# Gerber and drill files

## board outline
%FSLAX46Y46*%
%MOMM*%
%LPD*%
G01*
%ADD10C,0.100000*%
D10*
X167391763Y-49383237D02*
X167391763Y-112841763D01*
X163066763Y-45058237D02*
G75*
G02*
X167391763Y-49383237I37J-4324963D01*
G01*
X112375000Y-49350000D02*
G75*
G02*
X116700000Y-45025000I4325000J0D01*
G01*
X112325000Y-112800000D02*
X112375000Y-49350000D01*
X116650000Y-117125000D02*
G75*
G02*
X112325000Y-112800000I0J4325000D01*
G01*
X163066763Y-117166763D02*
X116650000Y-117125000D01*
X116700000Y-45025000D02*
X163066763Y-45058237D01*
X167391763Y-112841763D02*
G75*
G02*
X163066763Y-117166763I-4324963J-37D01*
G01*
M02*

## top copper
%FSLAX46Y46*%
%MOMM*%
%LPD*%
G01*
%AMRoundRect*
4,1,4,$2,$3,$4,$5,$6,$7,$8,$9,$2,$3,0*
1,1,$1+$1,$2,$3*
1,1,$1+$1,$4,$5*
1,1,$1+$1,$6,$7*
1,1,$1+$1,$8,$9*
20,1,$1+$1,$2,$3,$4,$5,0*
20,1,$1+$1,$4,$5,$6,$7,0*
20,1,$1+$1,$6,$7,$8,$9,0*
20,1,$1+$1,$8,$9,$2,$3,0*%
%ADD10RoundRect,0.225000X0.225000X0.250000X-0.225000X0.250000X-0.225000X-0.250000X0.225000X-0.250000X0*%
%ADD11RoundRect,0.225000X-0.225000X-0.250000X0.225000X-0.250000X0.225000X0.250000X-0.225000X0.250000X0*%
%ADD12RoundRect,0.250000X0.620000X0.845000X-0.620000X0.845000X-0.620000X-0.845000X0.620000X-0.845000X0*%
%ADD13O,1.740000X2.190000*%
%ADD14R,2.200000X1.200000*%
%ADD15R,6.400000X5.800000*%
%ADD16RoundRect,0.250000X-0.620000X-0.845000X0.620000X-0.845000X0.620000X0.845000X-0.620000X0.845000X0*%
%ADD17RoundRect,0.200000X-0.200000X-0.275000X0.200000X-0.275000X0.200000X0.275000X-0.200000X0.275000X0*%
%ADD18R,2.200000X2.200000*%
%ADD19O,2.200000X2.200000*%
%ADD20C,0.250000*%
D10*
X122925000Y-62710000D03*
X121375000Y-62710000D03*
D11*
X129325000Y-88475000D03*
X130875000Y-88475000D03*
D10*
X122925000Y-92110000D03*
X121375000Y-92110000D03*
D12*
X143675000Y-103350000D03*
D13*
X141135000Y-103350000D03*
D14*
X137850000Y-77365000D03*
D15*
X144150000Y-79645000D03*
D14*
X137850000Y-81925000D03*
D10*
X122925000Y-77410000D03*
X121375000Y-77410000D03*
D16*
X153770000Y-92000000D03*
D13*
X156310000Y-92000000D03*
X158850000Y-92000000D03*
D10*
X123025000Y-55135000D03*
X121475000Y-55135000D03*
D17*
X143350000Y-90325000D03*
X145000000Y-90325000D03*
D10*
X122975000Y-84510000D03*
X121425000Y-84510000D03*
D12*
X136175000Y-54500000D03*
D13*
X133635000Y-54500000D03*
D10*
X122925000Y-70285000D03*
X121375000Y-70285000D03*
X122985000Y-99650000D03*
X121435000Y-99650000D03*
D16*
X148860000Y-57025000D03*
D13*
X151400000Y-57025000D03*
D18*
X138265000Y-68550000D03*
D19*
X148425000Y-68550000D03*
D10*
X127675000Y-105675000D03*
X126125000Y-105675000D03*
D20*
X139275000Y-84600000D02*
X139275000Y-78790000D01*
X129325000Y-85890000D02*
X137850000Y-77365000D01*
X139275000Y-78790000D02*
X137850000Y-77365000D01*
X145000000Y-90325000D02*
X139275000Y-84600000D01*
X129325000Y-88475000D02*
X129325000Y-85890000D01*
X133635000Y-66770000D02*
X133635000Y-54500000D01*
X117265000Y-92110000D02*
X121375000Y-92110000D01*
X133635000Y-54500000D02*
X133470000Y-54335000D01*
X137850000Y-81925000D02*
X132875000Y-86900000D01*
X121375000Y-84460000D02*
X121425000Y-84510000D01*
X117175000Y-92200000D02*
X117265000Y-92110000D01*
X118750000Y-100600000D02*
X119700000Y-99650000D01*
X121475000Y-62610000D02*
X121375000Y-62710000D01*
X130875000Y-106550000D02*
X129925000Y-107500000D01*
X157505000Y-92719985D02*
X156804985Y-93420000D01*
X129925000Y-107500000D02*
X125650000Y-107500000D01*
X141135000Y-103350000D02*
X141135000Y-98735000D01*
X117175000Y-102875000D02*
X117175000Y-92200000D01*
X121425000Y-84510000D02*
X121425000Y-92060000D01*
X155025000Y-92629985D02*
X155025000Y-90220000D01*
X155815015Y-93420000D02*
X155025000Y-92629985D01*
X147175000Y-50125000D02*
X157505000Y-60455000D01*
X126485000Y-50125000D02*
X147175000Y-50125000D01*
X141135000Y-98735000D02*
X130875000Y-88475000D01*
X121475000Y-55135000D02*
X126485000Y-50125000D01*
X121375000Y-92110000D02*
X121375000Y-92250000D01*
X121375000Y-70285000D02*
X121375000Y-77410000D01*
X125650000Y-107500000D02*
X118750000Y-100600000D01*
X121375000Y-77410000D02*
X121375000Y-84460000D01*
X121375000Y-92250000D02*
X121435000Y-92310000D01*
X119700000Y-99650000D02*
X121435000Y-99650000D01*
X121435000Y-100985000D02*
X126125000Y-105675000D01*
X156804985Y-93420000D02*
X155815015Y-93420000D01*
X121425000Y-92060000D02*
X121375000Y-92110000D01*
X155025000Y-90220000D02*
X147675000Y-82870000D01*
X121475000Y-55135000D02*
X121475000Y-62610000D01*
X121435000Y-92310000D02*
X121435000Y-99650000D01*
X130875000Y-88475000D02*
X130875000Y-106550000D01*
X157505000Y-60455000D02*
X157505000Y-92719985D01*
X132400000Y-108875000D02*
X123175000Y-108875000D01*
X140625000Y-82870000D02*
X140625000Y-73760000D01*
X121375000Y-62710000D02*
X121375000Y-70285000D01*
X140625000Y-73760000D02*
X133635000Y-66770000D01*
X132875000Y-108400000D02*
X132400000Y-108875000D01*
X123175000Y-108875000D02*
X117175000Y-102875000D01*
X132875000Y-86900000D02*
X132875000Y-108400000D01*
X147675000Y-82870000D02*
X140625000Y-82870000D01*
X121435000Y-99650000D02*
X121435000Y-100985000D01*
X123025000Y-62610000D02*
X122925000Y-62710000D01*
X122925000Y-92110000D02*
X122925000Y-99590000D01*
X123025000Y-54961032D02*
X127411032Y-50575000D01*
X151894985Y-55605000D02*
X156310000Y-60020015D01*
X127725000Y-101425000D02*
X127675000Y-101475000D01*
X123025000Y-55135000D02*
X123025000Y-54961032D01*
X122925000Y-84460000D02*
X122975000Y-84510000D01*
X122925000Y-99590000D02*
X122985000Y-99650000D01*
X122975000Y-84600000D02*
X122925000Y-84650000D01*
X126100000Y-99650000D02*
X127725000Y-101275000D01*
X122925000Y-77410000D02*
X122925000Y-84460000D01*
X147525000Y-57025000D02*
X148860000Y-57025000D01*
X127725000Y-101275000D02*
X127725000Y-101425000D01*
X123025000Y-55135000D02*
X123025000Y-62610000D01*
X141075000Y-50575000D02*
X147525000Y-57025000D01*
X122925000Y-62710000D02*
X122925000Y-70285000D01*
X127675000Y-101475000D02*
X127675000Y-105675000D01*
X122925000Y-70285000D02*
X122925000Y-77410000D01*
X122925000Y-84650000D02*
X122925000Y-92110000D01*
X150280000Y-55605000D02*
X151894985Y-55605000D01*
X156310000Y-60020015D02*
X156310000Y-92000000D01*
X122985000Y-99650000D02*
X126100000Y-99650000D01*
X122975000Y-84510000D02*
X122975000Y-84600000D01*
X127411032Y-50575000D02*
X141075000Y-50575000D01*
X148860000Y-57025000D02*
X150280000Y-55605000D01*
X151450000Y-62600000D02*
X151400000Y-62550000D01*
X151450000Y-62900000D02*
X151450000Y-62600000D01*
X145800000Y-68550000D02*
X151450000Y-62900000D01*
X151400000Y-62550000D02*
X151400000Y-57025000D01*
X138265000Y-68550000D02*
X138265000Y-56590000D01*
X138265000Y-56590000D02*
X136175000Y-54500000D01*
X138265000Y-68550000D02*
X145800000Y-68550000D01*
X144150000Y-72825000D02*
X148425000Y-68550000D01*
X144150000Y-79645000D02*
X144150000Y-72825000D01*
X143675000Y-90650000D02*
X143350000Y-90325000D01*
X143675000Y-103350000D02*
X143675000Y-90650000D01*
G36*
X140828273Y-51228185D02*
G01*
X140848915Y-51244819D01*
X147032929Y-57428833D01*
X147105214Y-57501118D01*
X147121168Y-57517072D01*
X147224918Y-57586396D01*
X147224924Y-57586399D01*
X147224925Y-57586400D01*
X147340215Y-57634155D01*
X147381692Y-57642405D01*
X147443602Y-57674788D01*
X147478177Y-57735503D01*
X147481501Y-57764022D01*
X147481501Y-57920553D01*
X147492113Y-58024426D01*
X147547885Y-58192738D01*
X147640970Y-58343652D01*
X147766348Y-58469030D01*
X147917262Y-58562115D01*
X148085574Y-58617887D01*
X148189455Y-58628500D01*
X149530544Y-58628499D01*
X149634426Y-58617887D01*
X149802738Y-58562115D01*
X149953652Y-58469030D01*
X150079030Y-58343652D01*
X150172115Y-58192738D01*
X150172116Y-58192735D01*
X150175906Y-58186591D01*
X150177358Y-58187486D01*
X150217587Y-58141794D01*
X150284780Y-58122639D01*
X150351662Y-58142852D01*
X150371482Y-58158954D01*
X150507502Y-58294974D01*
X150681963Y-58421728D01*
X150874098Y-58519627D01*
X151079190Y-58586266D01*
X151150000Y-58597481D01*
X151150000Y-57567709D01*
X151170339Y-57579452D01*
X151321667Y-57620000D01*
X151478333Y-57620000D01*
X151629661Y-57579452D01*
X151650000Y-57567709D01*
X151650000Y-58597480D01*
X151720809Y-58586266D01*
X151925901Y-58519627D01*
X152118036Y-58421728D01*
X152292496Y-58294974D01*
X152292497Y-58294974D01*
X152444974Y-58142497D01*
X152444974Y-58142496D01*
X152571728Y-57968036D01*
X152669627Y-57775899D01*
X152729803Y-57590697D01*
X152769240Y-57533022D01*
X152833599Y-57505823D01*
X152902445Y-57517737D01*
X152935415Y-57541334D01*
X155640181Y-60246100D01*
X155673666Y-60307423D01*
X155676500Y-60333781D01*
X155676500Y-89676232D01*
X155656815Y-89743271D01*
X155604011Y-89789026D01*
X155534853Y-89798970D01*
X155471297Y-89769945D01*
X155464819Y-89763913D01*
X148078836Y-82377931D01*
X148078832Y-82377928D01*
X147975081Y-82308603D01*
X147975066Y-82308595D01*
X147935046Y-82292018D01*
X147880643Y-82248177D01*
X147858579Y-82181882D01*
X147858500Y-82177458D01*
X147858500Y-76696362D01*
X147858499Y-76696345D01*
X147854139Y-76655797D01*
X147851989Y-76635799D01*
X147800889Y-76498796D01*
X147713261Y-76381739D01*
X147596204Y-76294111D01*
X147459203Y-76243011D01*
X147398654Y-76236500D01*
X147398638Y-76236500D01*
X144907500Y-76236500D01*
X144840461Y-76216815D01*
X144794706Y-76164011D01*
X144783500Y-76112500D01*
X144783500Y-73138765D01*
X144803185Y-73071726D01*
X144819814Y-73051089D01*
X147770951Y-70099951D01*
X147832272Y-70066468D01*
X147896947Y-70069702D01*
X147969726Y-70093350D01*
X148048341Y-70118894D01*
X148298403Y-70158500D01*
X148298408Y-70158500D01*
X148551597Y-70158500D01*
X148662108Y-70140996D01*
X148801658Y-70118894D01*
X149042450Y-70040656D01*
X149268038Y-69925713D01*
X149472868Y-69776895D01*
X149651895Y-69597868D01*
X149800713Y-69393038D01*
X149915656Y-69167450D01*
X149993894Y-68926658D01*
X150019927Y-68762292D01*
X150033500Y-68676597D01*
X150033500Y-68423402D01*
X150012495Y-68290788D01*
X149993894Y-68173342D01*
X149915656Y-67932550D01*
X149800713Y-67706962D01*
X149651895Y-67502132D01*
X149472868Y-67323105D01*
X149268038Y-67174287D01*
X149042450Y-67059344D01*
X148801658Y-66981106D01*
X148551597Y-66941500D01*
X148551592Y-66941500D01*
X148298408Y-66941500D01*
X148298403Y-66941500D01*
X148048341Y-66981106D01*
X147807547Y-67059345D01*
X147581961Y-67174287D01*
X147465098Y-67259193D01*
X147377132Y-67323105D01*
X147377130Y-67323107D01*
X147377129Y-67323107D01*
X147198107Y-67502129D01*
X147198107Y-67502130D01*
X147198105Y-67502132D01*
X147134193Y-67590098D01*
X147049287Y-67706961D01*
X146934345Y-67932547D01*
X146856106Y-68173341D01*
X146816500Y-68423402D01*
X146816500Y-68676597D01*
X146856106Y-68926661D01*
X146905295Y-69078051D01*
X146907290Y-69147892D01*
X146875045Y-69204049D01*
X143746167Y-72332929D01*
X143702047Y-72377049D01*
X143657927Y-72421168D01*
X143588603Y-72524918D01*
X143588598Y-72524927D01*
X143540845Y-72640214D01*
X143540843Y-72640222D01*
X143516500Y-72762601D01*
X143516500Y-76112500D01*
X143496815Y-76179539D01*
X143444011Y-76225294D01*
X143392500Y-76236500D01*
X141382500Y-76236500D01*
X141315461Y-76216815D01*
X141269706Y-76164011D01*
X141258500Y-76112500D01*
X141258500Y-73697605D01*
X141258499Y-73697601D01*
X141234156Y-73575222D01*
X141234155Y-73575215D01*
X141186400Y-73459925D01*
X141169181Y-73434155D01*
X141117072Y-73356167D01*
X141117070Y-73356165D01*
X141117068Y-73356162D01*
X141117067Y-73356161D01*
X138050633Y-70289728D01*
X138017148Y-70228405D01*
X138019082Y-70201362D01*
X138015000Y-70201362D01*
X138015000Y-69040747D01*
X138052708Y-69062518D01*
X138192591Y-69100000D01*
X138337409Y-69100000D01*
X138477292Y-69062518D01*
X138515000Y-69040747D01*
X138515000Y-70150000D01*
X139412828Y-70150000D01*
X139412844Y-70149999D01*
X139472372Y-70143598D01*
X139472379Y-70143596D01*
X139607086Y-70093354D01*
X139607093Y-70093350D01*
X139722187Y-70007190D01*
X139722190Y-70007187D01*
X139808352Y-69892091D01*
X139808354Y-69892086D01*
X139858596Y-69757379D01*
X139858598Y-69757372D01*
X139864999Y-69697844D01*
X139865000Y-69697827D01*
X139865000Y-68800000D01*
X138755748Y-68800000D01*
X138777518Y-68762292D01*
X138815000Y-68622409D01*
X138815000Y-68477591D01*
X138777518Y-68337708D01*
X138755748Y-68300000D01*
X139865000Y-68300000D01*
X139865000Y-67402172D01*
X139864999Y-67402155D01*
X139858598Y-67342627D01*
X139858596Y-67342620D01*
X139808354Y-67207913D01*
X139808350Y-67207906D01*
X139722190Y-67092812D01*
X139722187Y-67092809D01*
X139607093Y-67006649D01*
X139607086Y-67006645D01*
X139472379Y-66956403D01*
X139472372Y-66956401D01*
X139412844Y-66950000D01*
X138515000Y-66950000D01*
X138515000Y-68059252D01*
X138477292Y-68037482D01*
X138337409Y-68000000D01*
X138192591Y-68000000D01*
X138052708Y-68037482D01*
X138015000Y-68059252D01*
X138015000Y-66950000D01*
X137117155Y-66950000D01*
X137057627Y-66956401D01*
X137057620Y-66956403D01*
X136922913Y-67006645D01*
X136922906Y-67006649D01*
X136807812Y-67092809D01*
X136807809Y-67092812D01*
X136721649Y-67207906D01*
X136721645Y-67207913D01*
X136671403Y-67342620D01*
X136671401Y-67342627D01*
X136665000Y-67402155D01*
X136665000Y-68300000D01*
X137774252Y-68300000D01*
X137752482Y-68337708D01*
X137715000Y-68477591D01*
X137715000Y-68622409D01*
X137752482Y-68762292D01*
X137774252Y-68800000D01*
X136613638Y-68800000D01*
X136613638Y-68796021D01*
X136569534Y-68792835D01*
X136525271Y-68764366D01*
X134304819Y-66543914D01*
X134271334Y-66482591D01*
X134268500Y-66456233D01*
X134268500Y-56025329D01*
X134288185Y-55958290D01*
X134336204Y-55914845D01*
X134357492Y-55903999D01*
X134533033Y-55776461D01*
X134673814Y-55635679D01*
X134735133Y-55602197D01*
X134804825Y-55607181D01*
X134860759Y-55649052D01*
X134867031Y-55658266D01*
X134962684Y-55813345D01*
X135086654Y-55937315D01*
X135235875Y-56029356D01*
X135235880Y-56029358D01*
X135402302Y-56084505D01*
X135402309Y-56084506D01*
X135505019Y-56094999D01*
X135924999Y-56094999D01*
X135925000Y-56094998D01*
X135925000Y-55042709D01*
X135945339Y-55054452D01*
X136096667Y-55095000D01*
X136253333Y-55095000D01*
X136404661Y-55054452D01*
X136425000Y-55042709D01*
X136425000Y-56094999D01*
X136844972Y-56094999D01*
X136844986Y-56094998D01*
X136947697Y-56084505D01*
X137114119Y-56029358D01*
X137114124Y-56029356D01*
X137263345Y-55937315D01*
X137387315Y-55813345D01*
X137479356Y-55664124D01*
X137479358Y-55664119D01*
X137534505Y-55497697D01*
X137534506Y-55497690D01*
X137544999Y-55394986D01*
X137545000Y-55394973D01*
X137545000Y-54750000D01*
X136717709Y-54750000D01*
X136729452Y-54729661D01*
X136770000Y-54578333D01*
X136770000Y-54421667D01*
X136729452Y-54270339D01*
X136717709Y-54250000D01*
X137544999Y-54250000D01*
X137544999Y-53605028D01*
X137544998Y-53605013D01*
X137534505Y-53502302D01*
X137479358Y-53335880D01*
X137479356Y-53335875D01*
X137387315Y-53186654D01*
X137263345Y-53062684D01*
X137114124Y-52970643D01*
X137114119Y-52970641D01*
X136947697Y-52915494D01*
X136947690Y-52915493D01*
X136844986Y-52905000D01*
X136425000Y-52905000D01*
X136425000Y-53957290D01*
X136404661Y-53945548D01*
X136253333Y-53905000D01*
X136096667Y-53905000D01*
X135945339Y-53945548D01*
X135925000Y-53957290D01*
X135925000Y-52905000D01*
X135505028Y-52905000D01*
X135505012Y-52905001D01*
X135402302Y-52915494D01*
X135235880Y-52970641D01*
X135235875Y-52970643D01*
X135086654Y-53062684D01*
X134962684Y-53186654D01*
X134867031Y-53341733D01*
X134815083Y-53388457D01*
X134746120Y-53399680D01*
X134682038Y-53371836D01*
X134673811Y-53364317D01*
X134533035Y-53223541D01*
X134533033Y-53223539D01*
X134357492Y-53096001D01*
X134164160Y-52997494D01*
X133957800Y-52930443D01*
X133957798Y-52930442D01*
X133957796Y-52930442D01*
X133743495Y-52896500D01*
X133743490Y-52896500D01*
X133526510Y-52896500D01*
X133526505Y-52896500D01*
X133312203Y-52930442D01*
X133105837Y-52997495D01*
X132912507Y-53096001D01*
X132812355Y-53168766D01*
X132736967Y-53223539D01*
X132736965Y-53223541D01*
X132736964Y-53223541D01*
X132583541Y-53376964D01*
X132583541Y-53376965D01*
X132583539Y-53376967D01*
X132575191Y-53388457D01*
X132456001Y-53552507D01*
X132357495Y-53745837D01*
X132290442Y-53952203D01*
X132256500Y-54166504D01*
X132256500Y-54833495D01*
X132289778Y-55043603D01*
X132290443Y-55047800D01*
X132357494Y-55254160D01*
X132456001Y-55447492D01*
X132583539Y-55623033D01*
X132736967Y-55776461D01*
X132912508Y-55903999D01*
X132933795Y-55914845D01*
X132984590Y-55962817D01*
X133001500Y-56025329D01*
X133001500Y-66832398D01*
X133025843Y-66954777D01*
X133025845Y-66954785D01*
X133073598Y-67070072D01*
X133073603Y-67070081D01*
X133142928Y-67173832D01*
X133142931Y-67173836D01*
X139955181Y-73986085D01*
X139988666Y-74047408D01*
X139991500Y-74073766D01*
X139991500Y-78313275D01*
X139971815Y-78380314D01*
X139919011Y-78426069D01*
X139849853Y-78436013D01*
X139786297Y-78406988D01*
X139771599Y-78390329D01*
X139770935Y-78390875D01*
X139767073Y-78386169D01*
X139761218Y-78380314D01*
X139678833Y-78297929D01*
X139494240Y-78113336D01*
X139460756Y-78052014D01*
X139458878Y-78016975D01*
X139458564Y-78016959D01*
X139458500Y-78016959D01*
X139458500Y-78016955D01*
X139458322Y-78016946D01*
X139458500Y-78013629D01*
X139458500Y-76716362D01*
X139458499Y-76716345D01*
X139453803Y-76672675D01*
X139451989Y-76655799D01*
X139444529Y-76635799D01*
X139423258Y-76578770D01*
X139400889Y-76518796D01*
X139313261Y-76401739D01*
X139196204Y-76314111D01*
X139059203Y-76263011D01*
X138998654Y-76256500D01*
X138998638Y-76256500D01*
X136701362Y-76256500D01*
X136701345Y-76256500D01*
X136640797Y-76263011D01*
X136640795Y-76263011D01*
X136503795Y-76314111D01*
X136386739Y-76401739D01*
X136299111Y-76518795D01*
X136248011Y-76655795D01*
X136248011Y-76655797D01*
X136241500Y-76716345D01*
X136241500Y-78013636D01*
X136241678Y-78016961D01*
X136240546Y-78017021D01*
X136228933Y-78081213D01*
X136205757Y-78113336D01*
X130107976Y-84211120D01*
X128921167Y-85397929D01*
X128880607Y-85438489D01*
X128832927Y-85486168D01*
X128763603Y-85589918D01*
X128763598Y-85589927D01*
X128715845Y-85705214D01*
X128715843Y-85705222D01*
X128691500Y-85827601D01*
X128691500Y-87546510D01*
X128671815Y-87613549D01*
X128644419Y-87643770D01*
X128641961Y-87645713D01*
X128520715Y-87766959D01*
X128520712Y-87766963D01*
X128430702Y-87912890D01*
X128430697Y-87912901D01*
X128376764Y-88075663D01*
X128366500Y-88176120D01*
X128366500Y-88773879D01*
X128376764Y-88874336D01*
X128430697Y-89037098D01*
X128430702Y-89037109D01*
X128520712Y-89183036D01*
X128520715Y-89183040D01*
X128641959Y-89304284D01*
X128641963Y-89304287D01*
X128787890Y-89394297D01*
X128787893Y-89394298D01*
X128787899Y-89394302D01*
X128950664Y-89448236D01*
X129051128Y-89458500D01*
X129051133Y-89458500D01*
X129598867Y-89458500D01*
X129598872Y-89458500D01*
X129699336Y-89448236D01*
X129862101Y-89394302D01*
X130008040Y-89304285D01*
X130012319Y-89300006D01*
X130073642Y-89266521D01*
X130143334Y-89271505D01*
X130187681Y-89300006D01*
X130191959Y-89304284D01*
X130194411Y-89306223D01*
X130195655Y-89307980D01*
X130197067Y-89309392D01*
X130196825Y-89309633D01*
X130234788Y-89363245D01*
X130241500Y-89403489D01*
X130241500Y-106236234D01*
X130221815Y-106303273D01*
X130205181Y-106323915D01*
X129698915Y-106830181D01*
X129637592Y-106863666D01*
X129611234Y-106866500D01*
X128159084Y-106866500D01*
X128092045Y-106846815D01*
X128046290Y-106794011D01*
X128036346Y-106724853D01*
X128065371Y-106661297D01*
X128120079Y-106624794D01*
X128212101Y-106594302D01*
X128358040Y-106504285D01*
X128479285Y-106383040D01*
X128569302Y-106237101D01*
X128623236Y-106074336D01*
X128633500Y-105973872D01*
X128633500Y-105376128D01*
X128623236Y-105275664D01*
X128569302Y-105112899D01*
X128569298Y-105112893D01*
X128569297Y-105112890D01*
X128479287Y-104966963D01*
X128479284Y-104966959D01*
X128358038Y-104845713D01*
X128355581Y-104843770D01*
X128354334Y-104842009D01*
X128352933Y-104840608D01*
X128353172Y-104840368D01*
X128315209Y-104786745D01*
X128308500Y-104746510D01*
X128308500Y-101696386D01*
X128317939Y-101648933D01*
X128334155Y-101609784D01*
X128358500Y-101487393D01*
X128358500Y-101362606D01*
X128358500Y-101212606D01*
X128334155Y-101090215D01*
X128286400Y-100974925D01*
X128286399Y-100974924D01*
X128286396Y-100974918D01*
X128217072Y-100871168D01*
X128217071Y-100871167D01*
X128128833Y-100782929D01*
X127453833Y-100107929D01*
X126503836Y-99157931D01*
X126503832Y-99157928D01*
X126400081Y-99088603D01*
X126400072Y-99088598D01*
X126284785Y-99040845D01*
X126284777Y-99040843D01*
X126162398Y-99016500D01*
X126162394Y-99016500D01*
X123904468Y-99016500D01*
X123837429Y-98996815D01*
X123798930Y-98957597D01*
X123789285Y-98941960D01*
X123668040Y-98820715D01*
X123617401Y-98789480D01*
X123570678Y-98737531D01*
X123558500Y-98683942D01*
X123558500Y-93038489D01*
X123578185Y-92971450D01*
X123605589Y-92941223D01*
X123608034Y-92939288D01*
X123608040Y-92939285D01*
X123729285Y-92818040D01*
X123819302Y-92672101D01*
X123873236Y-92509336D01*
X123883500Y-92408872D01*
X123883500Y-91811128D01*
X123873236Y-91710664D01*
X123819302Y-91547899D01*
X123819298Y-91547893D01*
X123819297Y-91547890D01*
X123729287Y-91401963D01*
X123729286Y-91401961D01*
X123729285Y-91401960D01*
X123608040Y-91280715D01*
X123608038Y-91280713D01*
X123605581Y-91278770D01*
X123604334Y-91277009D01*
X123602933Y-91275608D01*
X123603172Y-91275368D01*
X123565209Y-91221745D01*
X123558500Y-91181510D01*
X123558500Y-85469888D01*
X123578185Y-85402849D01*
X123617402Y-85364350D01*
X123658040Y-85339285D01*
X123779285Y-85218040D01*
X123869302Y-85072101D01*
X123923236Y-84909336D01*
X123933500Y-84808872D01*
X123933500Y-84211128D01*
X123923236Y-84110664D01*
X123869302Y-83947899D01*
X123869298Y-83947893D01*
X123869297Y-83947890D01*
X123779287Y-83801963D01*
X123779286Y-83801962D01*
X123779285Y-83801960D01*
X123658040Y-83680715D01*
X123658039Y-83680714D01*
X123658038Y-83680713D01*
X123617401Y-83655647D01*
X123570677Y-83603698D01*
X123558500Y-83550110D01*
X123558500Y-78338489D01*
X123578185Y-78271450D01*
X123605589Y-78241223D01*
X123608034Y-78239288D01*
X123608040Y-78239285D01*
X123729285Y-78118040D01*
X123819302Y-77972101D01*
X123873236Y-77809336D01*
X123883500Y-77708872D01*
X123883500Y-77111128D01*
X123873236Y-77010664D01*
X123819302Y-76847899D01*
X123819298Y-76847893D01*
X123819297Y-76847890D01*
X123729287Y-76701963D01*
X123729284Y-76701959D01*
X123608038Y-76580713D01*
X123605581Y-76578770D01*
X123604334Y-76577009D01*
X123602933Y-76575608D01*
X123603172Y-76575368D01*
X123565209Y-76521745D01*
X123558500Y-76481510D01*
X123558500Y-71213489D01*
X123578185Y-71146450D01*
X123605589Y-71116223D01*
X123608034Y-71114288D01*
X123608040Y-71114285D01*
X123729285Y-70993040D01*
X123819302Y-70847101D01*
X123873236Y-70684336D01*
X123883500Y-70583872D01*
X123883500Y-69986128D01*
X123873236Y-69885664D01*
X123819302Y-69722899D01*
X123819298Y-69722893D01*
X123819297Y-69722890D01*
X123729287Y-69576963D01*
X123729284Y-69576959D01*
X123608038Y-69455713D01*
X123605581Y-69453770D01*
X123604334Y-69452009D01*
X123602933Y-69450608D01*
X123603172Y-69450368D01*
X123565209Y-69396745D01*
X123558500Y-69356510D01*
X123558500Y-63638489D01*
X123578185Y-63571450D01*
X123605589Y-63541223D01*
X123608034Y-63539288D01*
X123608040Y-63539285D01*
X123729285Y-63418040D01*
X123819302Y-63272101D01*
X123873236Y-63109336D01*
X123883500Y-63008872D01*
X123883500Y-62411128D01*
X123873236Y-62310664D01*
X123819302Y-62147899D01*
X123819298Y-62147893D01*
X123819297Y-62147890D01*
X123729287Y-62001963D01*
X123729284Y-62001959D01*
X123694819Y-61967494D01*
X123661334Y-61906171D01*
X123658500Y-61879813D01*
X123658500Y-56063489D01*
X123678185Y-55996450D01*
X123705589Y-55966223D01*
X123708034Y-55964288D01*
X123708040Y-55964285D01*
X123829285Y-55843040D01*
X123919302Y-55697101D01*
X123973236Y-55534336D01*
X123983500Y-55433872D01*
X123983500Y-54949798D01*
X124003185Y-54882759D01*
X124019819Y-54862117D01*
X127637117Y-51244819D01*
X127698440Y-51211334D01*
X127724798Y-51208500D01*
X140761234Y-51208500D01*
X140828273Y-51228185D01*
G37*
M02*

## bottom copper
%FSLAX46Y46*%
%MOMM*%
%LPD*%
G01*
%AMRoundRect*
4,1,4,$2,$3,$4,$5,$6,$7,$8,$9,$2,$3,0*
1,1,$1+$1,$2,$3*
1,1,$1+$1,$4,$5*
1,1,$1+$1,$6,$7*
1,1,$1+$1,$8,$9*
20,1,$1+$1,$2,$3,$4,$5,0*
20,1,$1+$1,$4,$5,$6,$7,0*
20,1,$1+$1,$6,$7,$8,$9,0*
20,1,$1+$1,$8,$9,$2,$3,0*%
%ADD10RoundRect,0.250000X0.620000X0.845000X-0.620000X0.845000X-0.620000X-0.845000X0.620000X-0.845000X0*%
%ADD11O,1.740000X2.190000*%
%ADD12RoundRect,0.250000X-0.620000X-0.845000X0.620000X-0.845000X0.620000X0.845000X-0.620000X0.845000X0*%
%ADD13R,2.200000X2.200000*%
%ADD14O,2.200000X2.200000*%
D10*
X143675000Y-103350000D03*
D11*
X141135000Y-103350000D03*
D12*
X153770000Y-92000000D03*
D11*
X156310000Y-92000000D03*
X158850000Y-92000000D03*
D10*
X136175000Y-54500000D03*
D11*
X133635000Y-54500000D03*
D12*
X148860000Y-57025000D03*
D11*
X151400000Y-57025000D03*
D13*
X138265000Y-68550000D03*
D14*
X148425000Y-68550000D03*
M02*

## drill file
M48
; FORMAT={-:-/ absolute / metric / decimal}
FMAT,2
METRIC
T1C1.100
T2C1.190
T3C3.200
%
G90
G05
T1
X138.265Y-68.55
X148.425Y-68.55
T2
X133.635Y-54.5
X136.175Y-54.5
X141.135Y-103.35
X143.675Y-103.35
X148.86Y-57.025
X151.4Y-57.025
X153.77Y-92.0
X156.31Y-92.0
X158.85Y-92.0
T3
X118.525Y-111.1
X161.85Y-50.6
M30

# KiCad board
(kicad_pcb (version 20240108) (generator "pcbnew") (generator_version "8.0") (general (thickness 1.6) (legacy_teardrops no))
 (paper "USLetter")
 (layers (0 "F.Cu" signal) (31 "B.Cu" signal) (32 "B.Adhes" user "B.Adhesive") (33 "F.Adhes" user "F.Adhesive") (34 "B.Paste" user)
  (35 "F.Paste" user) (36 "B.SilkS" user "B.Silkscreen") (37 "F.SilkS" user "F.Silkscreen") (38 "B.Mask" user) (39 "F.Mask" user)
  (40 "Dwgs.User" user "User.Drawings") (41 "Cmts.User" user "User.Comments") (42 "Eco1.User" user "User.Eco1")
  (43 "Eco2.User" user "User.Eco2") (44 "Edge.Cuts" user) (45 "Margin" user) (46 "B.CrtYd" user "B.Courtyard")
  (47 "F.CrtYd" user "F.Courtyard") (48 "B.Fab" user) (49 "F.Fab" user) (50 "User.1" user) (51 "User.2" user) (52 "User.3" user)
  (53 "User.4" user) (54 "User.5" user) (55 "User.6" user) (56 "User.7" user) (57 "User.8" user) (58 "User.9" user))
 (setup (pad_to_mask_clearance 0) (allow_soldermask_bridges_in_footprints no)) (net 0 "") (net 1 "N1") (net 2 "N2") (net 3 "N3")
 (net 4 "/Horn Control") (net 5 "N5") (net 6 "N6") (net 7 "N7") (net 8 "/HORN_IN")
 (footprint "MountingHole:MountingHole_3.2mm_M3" (layer "F.Cu") (at 161.85 50.6)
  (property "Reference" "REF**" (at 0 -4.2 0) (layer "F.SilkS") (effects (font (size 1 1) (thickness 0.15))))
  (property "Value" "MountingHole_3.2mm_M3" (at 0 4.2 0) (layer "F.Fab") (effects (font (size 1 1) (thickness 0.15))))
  (pad "" np_thru_hole circle (at 0 0) (size 3.2 3.2) (drill 3.2) (layers "*.Cu" "*.Mask")))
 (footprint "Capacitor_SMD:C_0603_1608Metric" (layer "F.Cu") (at 122.15 62.71 180)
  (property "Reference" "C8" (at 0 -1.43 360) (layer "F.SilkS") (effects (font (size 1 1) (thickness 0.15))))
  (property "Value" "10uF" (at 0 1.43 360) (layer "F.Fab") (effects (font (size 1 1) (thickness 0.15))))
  (pad "1" smd roundrect (at -0.775 0 180) (size 0.9 0.95) (layers "F.Cu" "F.Paste" "F.Mask") (roundrect_rratio 0.25) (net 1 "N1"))
  (pad "2" smd roundrect (at 0.775 0 180) (size 0.9 0.95) (layers "F.Cu" "F.Paste" "F.Mask") (roundrect_rratio 0.25) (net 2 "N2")))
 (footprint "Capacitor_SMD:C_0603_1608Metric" (layer "F.Cu") (at 130.1 88.475)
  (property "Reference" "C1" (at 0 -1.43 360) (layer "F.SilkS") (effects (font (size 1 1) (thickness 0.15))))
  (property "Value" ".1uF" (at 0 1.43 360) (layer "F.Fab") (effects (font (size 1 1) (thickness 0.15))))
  (pad "1" smd roundrect (at -0.775 0) (size 0.9 0.95) (layers "F.Cu" "F.Paste" "F.Mask") (roundrect_rratio 0.25) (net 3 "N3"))
  (pad "2" smd roundrect (at 0.775 0) (size 0.9 0.95) (layers "F.Cu" "F.Paste" "F.Mask") (roundrect_rratio 0.25) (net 2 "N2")))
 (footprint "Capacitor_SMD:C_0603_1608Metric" (layer "F.Cu") (at 122.15 92.11 180)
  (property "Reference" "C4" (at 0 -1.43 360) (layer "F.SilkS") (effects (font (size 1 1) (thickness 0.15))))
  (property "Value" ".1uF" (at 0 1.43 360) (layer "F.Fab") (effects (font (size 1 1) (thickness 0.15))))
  (pad "1" smd roundrect (at -0.775 0 180) (size 0.9 0.95) (layers "F.Cu" "F.Paste" "F.Mask") (roundrect_rratio 0.25) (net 1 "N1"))
  (pad "2" smd roundrect (at 0.775 0 180) (size 0.9 0.95) (layers "F.Cu" "F.Paste" "F.Mask") (roundrect_rratio 0.25) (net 2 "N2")))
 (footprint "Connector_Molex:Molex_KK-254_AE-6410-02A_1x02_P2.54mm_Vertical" (layer "F.Cu") (at 143.675 103.35 180)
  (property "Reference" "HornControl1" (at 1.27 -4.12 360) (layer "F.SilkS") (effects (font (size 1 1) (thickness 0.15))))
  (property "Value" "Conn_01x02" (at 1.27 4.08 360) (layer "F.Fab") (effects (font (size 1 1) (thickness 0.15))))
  (pad "1" thru_hole roundrect (at 0 0 180) (size 1.74 2.19) (drill 1.19) (layers "*.Cu" "*.Mask") (remove_unused_layers no)
   (roundrect_rratio 0.143678) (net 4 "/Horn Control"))
  (pad "2" thru_hole oval (at 2.54 0 180) (size 1.74 2.19) (drill 1.19) (layers "*.Cu" "*.Mask") (remove_unused_layers no) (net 2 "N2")))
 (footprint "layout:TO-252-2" (layer "F.Cu") (at 142.05 79.645)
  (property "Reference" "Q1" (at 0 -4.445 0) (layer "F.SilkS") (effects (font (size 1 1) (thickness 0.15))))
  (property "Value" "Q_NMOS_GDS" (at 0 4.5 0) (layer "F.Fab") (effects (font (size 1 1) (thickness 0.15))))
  (pad "1" smd rect (at -4.2 -2.28) (size 2.2 1.2) (layers "F.Cu" "F.Paste" "F.Mask") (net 3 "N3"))
  (pad "2" smd rect (at 2.1 0) (size 6.4 5.8) (layers "F.Cu" "F.Mask") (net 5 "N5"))
  (pad "3" smd rect (at -4.2 2.28) (size 2.2 1.2) (layers "F.Cu" "F.Paste" "F.Mask") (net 2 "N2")))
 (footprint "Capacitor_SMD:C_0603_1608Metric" (layer "F.Cu") (at 122.15 77.41 180)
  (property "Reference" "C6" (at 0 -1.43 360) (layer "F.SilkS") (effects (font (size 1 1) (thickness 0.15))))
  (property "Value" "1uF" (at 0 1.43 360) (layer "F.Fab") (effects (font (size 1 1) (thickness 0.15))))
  (pad "1" smd roundrect (at -0.775 0 180) (size 0.9 0.95) (layers "F.Cu" "F.Paste" "F.Mask") (roundrect_rratio 0.25) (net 1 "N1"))
  (pad "2" smd roundrect (at 0.775 0 180) (size 0.9 0.95) (layers "F.Cu" "F.Paste" "F.Mask") (roundrect_rratio 0.25) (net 2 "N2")))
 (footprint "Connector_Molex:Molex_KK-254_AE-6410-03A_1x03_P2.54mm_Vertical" (layer "F.Cu") (at 153.77 92)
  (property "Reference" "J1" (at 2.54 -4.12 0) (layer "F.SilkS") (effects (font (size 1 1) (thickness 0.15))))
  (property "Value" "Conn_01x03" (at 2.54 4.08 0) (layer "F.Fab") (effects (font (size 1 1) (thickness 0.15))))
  (pad "1" thru_hole roundrect (at 0 0) (size 1.74 2.19) (drill 1.19) (layers "*.Cu" "*.Mask") (remove_unused_layers no)
   (roundrect_rratio 0.143678) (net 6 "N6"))
  (pad "2" thru_hole oval (at 2.54 0) (size 1.74 2.19) (drill 1.19) (layers "*.Cu" "*.Mask") (remove_unused_layers no) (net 1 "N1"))
  (pad "3" thru_hole oval (at 5.08 0) (size 1.74 2.19) (drill 1.19) (layers "*.Cu" "*.Mask") (remove_unused_layers no) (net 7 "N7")))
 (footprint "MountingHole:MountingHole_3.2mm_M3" (layer "F.Cu") (at 118.525 111.1)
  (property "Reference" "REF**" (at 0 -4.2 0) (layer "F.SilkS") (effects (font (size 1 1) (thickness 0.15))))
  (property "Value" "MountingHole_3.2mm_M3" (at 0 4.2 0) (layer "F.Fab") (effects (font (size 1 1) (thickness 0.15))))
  (pad "" np_thru_hole circle (at 0 0) (size 3.2 3.2) (drill 3.2) (layers "*.Cu" "*.Mask")))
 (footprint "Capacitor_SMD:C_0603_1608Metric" (layer "F.Cu") (at 122.25 55.135 180)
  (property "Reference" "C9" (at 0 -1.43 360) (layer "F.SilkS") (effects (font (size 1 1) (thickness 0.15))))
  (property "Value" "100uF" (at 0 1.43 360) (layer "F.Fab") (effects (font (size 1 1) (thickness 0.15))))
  (pad "1" smd roundrect (at -0.775 0 180) (size 0.9 0.95) (layers "F.Cu" "F.Paste" "F.Mask") (roundrect_rratio 0.25) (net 1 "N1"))
  (pad "2" smd roundrect (at 0.775 0 180) (size 0.9 0.95) (layers "F.Cu" "F.Paste" "F.Mask") (roundrect_rratio 0.25) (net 2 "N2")))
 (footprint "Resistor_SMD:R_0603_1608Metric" (layer "F.Cu") (at 144.175 90.325)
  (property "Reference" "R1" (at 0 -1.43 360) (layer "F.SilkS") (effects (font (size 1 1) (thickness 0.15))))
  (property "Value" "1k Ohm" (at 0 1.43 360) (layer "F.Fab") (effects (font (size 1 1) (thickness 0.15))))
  (pad "1" smd roundrect (at -0.825 0) (size 0.8 0.95) (layers "F.Cu" "F.Paste" "F.Mask") (roundrect_rratio 0.25) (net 4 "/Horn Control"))
  (pad "2" smd roundrect (at 0.825 0) (size 0.8 0.95) (layers "F.Cu" "F.Paste" "F.Mask") (roundrect_rratio 0.25) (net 3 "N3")))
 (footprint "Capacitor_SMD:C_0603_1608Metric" (layer "F.Cu") (at 122.2 84.51 180)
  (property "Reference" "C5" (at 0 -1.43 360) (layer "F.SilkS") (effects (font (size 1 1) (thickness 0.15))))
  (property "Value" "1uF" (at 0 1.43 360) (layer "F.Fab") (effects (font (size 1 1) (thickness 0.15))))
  (pad "1" smd roundrect (at -0.775 0 180) (size 0.9 0.95) (layers "F.Cu" "F.Paste" "F.Mask") (roundrect_rratio 0.25) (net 1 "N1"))
  (pad "2" smd roundrect (at 0.775 0 180) (size 0.9 0.95) (layers "F.Cu" "F.Paste" "F.Mask") (roundrect_rratio 0.25) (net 2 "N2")))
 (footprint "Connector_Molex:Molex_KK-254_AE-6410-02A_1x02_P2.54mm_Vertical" (layer "F.Cu") (at 136.175 54.5 180)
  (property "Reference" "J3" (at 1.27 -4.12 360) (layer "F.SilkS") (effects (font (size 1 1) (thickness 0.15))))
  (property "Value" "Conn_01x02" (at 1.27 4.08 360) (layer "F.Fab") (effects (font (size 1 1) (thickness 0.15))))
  (pad "1" thru_hole roundrect (at 0 0 180) (size 1.74 2.19) (drill 1.19) (layers "*.Cu" "*.Mask") (remove_unused_layers no)
   (roundrect_rratio 0.143678) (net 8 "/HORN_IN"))
  (pad "2" thru_hole oval (at 2.54 0 180) (size 1.74 2.19) (drill 1.19) (layers "*.Cu" "*.Mask") (remove_unused_layers no) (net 2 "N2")))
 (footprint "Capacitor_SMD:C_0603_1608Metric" (layer "F.Cu") (at 122.15 70.285 180)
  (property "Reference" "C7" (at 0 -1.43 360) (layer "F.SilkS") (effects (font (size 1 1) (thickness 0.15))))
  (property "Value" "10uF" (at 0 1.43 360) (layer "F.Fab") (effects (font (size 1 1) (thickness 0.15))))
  (pad "1" smd roundrect (at -0.775 0 180) (size 0.9 0.95) (layers "F.Cu" "F.Paste" "F.Mask") (roundrect_rratio 0.25) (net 1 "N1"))
  (pad "2" smd roundrect (at 0.775 0 180) (size 0.9 0.95) (layers "F.Cu" "F.Paste" "F.Mask") (roundrect_rratio 0.25) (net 2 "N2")))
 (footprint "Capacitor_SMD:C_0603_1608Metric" (layer "F.Cu") (at 122.21 99.65 180)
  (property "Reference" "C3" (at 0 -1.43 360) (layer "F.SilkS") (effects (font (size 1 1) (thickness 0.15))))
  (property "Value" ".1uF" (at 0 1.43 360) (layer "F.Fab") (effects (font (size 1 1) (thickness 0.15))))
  (pad "1" smd roundrect (at -0.775 0 180) (size 0.9 0.95) (layers "F.Cu" "F.Paste" "F.Mask") (roundrect_rratio 0.25) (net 1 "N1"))
  (pad "2" smd roundrect (at 0.775 0 180) (size 0.9 0.95) (layers "F.Cu" "F.Paste" "F.Mask") (roundrect_rratio 0.25) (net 2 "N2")))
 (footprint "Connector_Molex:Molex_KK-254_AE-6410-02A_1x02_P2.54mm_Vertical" (layer "F.Cu") (at 148.86 57.025)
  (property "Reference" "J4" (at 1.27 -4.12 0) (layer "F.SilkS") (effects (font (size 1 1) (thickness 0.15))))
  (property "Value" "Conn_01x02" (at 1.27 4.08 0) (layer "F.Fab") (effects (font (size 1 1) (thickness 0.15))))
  (pad "1" thru_hole roundrect (at 0 0) (size 1.74 2.19) (drill 1.19) (layers "*.Cu" "*.Mask") (remove_unused_layers no)
   (roundrect_rratio 0.143678) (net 1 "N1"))
  (pad "2" thru_hole oval (at 2.54 0) (size 1.74 2.19) (drill 1.19) (layers "*.Cu" "*.Mask") (remove_unused_layers no) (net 8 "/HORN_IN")))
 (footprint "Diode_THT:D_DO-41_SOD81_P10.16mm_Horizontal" (layer "F.Cu") (at 138.265 68.55)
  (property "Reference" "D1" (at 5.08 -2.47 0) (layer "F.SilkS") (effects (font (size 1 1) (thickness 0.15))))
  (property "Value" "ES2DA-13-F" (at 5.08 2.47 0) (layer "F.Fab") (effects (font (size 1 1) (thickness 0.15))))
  (pad "1" thru_hole rect (at 0 0) (size 2.2 2.2) (drill 1.1) (layers "*.Cu" "*.Mask") (remove_unused_layers no) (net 8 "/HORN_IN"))
  (pad "2" thru_hole oval (at 10.16 0) (size 2.2 2.2) (drill 1.1) (layers "*.Cu" "*.Mask") (remove_unused_layers no) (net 5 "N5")))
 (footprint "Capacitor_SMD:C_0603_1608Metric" (layer "F.Cu") (at 126.9 105.675 180)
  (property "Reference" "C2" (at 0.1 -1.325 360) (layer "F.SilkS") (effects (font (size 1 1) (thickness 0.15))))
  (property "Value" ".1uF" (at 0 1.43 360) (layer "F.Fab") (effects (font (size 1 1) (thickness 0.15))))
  (pad "1" smd roundrect (at -0.775 0 180) (size 0.9 0.95) (layers "F.Cu" "F.Paste" "F.Mask") (roundrect_rratio 0.25) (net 1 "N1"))
  (pad "2" smd roundrect (at 0.775 0 180) (size 0.9 0.95) (layers "F.Cu" "F.Paste" "F.Mask") (roundrect_rratio 0.25) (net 2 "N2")))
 (gr_line (start 167.391763 49.383237) (end 167.391763 112.841763) (stroke (width 0.1) (type default)) (layer "Edge.Cuts"))
 (gr_arc (start 163.066763 45.058237) (mid 166.125 46.325) (end 167.391763 49.383237) (stroke (width 0.1) (type default))
  (layer "Edge.Cuts"))
 (gr_arc (start 112.375 49.35) (mid 113.641763 46.291763) (end 116.7 45.025) (stroke (width 0.1) (type default)) (layer "Edge.Cuts"))
 (gr_line (start 112.325 112.8) (end 112.375 49.35) (stroke (width 0.1) (type default)) (layer "Edge.Cuts"))
 (gr_arc (start 116.65 117.125) (mid 113.591763 115.858237) (end 112.325 112.8) (stroke (width 0.1) (type default)) (layer "Edge.Cuts"))
 (gr_line (start 163.066763 117.166763) (end 116.65 117.125) (stroke (width 0.1) (type default)) (layer "Edge.Cuts"))
 (gr_line (start 116.7 45.025) (end 163.066763 45.058237) (stroke (width 0.1) (type default)) (layer "Edge.Cuts"))
 (gr_arc (start 167.391763 112.841763) (mid 166.125 115.9) (end 163.066763 117.166763) (stroke (width 0.1) (type default))
  (layer "Edge.Cuts"))
 (segment (start 139.275 84.6) (end 139.275 78.79) (width 0.25) (layer "F.Cu") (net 3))
 (segment (start 129.325 85.89) (end 137.85 77.365) (width 0.25) (layer "F.Cu") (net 3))
 (segment (start 139.275 78.79) (end 137.85 77.365) (width 0.25) (layer "F.Cu") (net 3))
 (segment (start 145 90.325) (end 139.275 84.6) (width 0.25) (layer "F.Cu") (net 3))
 (segment (start 129.325 88.475) (end 129.325 85.89) (width 0.25) (layer "F.Cu") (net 3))
 (segment (start 133.635 66.77) (end 133.635 54.5) (width 0.25) (layer "F.Cu") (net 2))
 (segment (start 117.265 92.11) (end 121.375 92.11) (width 0.25) (layer "F.Cu") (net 2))
 (segment (start 133.635 54.5) (end 133.47 54.335) (width 0.25) (layer "F.Cu") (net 2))
 (segment (start 137.85 81.925) (end 132.875 86.9) (width 0.25) (layer "F.Cu") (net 2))
 (segment (start 121.375 84.46) (end 121.425 84.51) (width 0.25) (layer "F.Cu") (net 2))
 (segment (start 117.175 92.2) (end 117.265 92.11) (width 0.25) (layer "F.Cu") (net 2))
 (segment (start 118.75 100.6) (end 119.7 99.65) (width 0.25) (layer "F.Cu") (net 2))
 (segment (start 121.475 62.61) (end 121.375 62.71) (width 0.25) (layer "F.Cu") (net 2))
 (segment (start 130.875 106.55) (end 129.925 107.5) (width 0.25) (layer "F.Cu") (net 2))
 (segment (start 157.505 92.719985) (end 156.804985 93.42) (width 0.25) (layer "F.Cu") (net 2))
 (segment (start 129.925 107.5) (end 125.65 107.5) (width 0.25) (layer "F.Cu") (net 2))
 (segment (start 141.135 103.35) (end 141.135 98.735) (width 0.25) (layer "F.Cu") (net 2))
 (segment (start 117.175 102.875) (end 117.175 92.2) (width 0.25) (layer "F.Cu") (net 2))
 (segment (start 121.425 84.51) (end 121.425 92.06) (width 0.25) (layer "F.Cu") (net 2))
 (segment (start 155.025 92.629985) (end 155.025 90.22) (width 0.25) (layer "F.Cu") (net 2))
 (segment (start 155.815015 93.42) (end 155.025 92.629985) (width 0.25) (layer "F.Cu") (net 2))
 (segment (start 147.175 50.125) (end 157.505 60.455) (width 0.25) (layer "F.Cu") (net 2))
 (segment (start 126.485 50.125) (end 147.175 50.125) (width 0.25) (layer "F.Cu") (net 2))
 (segment (start 141.135 98.735) (end 130.875 88.475) (width 0.25) (layer "F.Cu") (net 2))
 (segment (start 121.475 55.135) (end 126.485 50.125) (width 0.25) (layer "F.Cu") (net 2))
 (segment (start 121.375 92.11) (end 121.375 92.25) (width 0.25) (layer "F.Cu") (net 2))
 (segment (start 121.375 70.285) (end 121.375 77.41) (width 0.25) (layer "F.Cu") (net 2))
 (segment (start 125.65 107.5) (end 118.75 100.6) (width 0.25) (layer "F.Cu") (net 2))
 (segment (start 121.375 77.41) (end 121.375 84.46) (width 0.25) (layer "F.Cu") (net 2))
 (segment (start 121.375 92.25) (end 121.435 92.31) (width 0.25) (layer "F.Cu") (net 2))
 (segment (start 119.7 99.65) (end 121.435 99.65) (width 0.25) (layer "F.Cu") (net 2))
 (segment (start 121.435 100.985) (end 126.125 105.675) (width 0.25) (layer "F.Cu") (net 2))
 (segment (start 156.804985 93.42) (end 155.815015 93.42) (width 0.25) (layer "F.Cu") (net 2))
 (segment (start 121.425 92.06) (end 121.375 92.11) (width 0.25) (layer "F.Cu") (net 2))
 (segment (start 155.025 90.22) (end 147.675 82.87) (width 0.25) (layer "F.Cu") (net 2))
 (segment (start 121.475 55.135) (end 121.475 62.61) (width 0.25) (layer "F.Cu") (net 2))
 (segment (start 121.435 92.31) (end 121.435 99.65) (width 0.25) (layer "F.Cu") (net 2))
 (segment (start 130.875 88.475) (end 130.875 106.55) (width 0.25) (layer "F.Cu") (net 2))
 (segment (start 157.505 60.455) (end 157.505 92.719985) (width 0.25) (layer "F.Cu") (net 2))
 (segment (start 132.4 108.875) (end 123.175 108.875) (width 0.25) (layer "F.Cu") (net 2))
 (segment (start 140.625 82.87) (end 140.625 73.76) (width 0.25) (layer "F.Cu") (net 2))
 (segment (start 121.375 62.71) (end 121.375 70.285) (width 0.25) (layer "F.Cu") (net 2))
 (segment (start 140.625 73.76) (end 133.635 66.77) (width 0.25) (layer "F.Cu") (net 2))
 (segment (start 132.875 108.4) (end 132.4 108.875) (width 0.25) (layer "F.Cu") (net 2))
 (segment (start 123.175 108.875) (end 117.175 102.875) (width 0.25) (layer "F.Cu") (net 2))
 (segment (start 132.875 86.9) (end 132.875 108.4) (width 0.25) (layer "F.Cu") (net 2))
 (segment (start 147.675 82.87) (end 140.625 82.87) (width 0.25) (layer "F.Cu") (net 2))
 (segment (start 121.435 99.65) (end 121.435 100.985) (width 0.25) (layer "F.Cu") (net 2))
 (segment (start 123.025 62.61) (end 122.925 62.71) (width 0.25) (layer "F.Cu") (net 1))
 (segment (start 122.925 92.11) (end 122.925 99.59) (width 0.25) (layer "F.Cu") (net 1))
 (segment (start 123.025 54.961032) (end 127.411032 50.575) (width 0.25) (layer "F.Cu") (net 1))
 (segment (start 151.894985 55.605) (end 156.31 60.020015) (width 0.25) (layer "F.Cu") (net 1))
 (segment (start 127.725 101.425) (end 127.675 101.475) (width 0.25) (layer "F.Cu") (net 1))
 (segment (start 123.025 55.135) (end 123.025 54.961032) (width 0.25) (layer "F.Cu") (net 1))
 (segment (start 122.925 84.46) (end 122.975 84.51) (width 0.25) (layer "F.Cu") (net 1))
 (segment (start 122.925 99.59) (end 122.985 99.65) (width 0.25) (layer "F.Cu") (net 1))
 (segment (start 122.975 84.6) (end 122.925 84.65) (width 0.25) (layer "F.Cu") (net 1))
 (segment (start 126.1 99.65) (end 127.725 101.275) (width 0.25) (layer "F.Cu") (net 1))
 (segment (start 122.925 77.41) (end 122.925 84.46) (width 0.25) (layer "F.Cu") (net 1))
 (segment (start 147.525 57.025) (end 148.86 57.025) (width 0.25) (layer "F.Cu") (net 1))
 (segment (start 127.725 101.275) (end 127.725 101.425) (width 0.25) (layer "F.Cu") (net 1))
 (segment (start 123.025 55.135) (end 123.025 62.61) (width 0.25) (layer "F.Cu") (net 1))
 (segment (start 141.075 50.575) (end 147.525 57.025) (width 0.25) (layer "F.Cu") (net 1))
 (segment (start 122.925 62.71) (end 122.925 70.285) (width 0.25) (layer "F.Cu") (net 1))
 (segment (start 127.675 101.475) (end 127.675 105.675) (width 0.25) (layer "F.Cu") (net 1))
 (segment (start 122.925 70.285) (end 122.925 77.41) (width 0.25) (layer "F.Cu") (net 1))
 (segment (start 122.925 84.65) (end 122.925 92.11) (width 0.25) (layer "F.Cu") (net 1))
 (segment (start 150.28 55.605) (end 151.894985 55.605) (width 0.25) (layer "F.Cu") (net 1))
 (segment (start 156.31 60.020015) (end 156.31 92) (width 0.25) (layer "F.Cu") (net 1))
 (segment (start 122.985 99.65) (end 126.1 99.65) (width 0.25) (layer "F.Cu") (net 1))
 (segment (start 122.975 84.51) (end 122.975 84.6) (width 0.25) (layer "F.Cu") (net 1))
 (segment (start 127.411032 50.575) (end 141.075 50.575) (width 0.25) (layer "F.Cu") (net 1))
 (segment (start 148.86 57.025) (end 150.28 55.605) (width 0.25) (layer "F.Cu") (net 1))
 (segment (start 151.45 62.6) (end 151.4 62.55) (width 0.25) (layer "F.Cu") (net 8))
 (segment (start 151.45 62.9) (end 151.45 62.6) (width 0.25) (layer "F.Cu") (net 8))
 (segment (start 145.8 68.55) (end 151.45 62.9) (width 0.25) (layer "F.Cu") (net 8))
 (segment (start 151.4 62.55) (end 151.4 57.025) (width 0.25) (layer "F.Cu") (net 8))
 (segment (start 138.265 68.55) (end 138.265 56.59) (width 0.25) (layer "F.Cu") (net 8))
 (segment (start 138.265 56.59) (end 136.175 54.5) (width 0.25) (layer "F.Cu") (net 8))
 (segment (start 138.265 68.55) (end 145.8 68.55) (width 0.25) (layer "F.Cu") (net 8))
 (segment (start 144.15 72.825) (end 148.425 68.55) (width 0.25) (layer "F.Cu") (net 5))
 (segment (start 144.15 79.645) (end 144.15 72.825) (width 0.25) (layer "F.Cu") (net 5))
 (segment (start 143.675 90.65) (end 143.35 90.325) (width 0.25) (layer "F.Cu") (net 4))
 (segment (start 143.675 103.35) (end 143.675 90.65) (width 0.25) (layer "F.Cu") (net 4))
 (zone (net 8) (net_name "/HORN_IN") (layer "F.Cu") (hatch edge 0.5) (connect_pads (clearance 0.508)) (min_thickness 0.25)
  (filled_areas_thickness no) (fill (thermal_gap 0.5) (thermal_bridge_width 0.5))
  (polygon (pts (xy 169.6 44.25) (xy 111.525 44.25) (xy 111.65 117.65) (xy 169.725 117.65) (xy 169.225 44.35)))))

